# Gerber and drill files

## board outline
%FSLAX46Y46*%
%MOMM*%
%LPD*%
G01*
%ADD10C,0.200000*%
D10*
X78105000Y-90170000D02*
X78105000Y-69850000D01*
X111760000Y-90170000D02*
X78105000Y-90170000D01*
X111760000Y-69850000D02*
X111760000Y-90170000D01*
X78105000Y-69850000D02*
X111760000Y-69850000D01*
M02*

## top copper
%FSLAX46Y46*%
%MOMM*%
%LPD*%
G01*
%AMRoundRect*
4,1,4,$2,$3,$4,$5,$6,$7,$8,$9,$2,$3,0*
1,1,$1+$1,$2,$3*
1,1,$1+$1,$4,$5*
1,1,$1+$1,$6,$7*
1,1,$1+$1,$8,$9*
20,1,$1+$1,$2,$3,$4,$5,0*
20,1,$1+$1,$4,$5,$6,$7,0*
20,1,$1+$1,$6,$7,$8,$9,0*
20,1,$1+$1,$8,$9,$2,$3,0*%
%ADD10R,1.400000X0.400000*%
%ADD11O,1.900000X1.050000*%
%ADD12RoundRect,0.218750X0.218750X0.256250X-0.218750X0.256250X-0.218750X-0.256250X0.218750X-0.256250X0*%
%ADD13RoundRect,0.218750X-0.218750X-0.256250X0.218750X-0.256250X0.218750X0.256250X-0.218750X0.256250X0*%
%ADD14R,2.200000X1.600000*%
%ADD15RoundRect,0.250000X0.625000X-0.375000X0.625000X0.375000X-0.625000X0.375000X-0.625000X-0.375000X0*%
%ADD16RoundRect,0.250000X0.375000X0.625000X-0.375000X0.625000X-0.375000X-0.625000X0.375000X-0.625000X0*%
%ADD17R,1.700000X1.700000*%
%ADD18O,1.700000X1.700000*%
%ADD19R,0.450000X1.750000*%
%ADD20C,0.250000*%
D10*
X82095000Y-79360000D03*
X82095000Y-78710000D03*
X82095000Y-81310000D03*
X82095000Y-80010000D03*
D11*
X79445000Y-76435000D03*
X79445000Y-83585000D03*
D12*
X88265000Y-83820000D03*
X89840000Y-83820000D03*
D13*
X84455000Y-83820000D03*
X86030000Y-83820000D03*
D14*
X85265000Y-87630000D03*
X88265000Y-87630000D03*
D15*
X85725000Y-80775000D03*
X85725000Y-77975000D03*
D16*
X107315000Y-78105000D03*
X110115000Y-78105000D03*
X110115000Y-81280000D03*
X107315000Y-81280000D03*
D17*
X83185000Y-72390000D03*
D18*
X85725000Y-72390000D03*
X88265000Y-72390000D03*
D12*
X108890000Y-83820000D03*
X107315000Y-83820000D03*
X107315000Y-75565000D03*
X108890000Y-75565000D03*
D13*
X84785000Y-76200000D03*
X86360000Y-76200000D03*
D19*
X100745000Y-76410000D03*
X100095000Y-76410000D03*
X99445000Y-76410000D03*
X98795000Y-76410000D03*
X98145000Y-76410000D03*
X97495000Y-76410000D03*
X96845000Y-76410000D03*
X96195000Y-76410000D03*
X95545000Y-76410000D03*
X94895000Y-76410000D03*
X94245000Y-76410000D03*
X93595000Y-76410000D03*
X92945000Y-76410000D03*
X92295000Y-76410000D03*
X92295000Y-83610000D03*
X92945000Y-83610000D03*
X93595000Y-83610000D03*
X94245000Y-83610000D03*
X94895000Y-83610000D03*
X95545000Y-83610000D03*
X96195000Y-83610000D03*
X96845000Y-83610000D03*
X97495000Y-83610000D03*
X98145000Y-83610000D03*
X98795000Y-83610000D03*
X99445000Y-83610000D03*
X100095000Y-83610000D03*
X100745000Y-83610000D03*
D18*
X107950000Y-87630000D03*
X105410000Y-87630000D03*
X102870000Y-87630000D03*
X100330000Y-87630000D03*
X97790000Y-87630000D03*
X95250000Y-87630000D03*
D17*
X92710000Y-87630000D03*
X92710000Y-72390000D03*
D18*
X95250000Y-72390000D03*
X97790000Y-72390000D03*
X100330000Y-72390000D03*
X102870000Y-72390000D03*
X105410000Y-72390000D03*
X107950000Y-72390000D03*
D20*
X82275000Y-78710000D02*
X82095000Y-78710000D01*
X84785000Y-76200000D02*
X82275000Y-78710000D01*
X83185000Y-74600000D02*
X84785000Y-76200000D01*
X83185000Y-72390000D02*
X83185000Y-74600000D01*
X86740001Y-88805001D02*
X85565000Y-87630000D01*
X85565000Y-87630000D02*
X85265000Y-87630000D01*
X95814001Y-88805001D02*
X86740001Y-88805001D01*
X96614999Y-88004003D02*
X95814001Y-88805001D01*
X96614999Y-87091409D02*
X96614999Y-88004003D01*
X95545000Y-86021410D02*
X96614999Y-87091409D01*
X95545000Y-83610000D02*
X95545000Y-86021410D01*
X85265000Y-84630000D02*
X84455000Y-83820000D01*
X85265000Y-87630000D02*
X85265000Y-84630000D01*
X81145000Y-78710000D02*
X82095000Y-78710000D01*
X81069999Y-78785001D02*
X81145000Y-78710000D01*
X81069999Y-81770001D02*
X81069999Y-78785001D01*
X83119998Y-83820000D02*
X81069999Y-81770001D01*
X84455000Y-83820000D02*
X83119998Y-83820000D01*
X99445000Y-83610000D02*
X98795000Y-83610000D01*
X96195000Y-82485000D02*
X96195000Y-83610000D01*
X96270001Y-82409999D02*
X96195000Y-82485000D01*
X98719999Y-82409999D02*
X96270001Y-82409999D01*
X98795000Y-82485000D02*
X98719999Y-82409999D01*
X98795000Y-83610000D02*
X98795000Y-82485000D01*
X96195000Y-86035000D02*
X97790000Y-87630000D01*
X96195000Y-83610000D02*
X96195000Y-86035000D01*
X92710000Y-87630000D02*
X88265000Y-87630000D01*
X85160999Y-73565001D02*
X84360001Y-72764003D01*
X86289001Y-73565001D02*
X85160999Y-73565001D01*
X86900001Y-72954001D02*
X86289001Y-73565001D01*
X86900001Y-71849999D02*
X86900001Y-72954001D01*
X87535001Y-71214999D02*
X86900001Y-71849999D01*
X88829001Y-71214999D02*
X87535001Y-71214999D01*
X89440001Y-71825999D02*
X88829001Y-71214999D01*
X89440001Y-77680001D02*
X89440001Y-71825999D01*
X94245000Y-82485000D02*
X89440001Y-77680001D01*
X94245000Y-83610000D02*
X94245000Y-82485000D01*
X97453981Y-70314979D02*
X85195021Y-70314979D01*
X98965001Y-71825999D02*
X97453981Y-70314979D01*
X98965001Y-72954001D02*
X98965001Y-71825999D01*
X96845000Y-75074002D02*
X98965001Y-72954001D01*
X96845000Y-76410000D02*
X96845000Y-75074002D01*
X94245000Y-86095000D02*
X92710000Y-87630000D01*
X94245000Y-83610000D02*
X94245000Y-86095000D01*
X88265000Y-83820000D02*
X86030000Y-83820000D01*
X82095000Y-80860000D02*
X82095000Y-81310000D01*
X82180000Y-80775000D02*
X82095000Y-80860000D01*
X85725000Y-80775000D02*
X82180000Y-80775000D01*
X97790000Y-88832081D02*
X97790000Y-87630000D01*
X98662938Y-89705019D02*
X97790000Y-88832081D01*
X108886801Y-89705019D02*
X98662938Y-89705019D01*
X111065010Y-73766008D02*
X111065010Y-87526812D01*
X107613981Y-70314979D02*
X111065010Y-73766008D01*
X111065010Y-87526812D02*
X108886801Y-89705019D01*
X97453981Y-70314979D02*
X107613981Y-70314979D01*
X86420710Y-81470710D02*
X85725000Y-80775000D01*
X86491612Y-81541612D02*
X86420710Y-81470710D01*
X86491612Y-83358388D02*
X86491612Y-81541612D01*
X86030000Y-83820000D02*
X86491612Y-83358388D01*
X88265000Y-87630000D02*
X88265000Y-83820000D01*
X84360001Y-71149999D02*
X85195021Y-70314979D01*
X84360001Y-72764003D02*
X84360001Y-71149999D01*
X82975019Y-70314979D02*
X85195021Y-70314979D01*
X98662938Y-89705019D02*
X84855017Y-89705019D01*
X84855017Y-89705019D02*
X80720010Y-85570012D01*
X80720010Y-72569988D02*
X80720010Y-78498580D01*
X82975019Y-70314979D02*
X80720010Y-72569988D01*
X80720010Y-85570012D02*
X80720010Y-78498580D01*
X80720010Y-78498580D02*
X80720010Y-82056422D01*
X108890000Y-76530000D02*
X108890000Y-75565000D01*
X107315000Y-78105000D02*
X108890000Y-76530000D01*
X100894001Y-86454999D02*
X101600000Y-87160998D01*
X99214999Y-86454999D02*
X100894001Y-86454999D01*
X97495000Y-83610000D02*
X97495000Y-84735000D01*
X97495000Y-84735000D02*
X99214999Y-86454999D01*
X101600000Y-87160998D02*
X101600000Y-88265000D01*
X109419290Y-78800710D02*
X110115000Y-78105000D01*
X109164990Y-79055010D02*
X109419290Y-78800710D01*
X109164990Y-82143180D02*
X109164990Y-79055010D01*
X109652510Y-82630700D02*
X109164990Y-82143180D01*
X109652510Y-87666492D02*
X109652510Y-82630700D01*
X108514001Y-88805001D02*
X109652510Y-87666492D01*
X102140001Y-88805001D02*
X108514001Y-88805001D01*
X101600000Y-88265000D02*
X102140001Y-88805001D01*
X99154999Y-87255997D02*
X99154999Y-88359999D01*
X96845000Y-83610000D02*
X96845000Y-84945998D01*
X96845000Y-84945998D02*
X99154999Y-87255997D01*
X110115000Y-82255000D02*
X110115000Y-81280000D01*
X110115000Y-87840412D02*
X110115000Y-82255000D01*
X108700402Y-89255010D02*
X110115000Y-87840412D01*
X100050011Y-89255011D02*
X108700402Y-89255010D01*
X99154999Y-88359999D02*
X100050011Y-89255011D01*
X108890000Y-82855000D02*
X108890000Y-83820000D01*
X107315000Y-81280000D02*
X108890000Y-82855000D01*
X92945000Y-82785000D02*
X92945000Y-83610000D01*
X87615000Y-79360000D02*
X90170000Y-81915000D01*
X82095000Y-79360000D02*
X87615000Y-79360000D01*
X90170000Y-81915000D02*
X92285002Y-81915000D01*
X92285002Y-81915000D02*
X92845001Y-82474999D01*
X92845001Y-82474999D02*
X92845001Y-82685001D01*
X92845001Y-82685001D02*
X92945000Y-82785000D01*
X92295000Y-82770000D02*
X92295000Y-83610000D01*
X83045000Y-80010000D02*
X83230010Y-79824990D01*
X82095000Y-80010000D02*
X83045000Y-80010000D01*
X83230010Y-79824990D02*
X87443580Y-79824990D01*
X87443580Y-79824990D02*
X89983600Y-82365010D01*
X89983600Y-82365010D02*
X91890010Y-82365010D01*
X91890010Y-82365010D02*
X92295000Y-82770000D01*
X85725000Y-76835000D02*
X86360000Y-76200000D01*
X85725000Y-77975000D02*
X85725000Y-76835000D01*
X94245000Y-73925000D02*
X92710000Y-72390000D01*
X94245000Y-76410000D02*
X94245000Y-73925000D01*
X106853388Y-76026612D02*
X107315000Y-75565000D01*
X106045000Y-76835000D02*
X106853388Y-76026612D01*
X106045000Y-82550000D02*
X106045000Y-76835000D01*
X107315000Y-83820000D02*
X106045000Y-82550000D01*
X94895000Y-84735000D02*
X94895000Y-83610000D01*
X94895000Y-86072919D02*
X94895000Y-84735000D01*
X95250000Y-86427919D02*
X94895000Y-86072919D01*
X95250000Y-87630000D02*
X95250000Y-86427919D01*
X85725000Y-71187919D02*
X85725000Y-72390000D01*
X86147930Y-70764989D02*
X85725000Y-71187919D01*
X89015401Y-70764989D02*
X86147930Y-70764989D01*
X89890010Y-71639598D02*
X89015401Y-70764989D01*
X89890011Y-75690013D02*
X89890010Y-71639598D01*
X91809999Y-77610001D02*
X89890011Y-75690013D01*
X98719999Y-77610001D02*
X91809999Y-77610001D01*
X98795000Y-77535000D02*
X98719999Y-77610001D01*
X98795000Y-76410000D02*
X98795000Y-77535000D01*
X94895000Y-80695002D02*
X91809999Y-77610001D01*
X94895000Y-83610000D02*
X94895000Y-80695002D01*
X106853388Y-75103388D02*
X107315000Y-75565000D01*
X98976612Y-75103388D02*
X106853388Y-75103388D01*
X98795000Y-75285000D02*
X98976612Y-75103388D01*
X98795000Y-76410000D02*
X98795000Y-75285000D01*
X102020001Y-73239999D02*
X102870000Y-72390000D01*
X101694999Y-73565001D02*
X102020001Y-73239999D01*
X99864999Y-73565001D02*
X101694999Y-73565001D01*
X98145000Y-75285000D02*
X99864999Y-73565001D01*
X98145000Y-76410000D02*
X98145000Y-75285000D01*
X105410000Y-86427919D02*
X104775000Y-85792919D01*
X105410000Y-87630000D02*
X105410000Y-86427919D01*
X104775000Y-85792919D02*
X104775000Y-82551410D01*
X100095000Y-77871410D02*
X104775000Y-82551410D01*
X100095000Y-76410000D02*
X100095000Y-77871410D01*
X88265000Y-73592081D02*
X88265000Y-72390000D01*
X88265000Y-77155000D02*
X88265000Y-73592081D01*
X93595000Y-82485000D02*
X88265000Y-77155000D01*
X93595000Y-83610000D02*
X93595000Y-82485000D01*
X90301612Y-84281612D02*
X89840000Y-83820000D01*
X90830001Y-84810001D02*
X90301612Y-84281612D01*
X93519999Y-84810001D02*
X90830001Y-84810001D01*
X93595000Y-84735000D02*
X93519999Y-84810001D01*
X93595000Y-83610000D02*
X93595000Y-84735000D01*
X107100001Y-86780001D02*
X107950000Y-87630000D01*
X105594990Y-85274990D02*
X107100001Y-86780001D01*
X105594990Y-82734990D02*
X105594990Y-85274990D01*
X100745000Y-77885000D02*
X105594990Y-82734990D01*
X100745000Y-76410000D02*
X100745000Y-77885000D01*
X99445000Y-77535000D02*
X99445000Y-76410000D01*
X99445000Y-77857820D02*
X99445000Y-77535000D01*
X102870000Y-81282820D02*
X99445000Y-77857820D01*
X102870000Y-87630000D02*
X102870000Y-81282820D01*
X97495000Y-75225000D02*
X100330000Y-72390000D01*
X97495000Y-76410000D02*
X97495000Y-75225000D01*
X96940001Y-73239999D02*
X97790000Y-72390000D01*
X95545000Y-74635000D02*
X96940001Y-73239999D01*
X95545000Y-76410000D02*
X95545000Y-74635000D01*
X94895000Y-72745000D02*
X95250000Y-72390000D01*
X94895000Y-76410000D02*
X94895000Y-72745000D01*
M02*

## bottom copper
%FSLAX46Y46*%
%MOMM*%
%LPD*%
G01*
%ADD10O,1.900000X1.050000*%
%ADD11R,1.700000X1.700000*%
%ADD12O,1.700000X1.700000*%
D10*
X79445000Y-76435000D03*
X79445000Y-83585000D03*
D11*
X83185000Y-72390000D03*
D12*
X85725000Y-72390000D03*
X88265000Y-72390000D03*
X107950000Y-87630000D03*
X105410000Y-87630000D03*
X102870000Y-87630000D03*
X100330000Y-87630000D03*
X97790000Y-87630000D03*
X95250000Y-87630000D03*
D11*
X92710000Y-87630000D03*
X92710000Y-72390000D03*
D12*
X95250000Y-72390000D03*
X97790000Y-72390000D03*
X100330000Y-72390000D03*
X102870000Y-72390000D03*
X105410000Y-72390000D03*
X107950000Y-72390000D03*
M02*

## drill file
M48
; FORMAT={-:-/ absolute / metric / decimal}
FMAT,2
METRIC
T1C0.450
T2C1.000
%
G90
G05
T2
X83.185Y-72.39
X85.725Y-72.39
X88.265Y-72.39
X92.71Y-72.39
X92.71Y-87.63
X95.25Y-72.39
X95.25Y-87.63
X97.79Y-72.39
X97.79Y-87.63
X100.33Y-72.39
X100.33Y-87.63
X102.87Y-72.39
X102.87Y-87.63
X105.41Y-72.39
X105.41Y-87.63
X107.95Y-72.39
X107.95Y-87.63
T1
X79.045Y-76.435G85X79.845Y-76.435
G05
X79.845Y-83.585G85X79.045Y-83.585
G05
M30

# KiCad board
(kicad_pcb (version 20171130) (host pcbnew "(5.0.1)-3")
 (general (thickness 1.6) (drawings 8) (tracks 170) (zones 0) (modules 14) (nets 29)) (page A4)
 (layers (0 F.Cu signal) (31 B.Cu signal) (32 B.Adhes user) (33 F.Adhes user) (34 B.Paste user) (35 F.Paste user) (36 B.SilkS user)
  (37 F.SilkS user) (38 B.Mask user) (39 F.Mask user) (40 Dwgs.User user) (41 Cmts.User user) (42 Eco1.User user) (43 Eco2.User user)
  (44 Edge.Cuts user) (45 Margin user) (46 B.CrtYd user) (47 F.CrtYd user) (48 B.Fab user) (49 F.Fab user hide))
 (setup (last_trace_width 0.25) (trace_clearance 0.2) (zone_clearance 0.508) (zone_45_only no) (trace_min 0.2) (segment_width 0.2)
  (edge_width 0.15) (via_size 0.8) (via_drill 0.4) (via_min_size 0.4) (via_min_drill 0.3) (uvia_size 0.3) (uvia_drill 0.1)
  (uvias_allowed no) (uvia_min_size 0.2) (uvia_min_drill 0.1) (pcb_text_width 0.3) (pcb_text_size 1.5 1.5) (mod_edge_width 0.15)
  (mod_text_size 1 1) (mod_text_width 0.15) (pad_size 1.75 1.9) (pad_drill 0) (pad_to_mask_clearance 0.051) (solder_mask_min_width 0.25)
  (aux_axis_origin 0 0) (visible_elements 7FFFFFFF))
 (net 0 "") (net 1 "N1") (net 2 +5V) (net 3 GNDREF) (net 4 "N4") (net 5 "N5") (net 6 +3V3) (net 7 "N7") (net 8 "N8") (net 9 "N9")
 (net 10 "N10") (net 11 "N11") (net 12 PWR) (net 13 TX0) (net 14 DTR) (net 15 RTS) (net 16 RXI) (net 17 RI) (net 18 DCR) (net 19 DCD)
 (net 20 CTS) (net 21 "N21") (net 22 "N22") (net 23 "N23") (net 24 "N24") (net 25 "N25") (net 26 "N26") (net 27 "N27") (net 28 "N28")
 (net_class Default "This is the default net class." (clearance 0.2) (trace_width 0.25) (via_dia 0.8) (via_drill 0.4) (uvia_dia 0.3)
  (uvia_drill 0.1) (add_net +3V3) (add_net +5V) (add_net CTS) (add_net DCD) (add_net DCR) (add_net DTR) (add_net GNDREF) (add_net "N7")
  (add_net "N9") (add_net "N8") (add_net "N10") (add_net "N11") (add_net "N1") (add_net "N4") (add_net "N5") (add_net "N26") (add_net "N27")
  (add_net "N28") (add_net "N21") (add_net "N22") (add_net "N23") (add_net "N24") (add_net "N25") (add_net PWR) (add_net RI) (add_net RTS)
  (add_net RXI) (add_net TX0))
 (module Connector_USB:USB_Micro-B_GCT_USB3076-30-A (layer F.Cu) (at 80.645 80.01 270)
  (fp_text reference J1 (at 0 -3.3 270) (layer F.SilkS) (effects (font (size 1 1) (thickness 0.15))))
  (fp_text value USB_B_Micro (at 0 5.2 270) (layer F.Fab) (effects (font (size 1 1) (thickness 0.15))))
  (pad 2 smd rect (at -0.65 -1.45 270) (size 0.4 1.4) (layers F.Cu F.Paste F.Mask) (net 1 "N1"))
  (pad 1 smd rect (at -1.3 -1.45 270) (size 0.4 1.4) (layers F.Cu F.Paste F.Mask) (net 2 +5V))
  (pad 5 smd rect (at 1.3 -1.45 270) (size 0.4 1.4) (layers F.Cu F.Paste F.Mask) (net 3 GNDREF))
  (pad 3 smd rect (at 0 -1.45 270) (size 0.4 1.4) (layers F.Cu F.Paste F.Mask) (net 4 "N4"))
  (pad 6 thru_hole oval (at -3.575 1.2 90) (size 1.05 1.9) (drill oval 0.45 1.25) (layers *.Cu *.Mask) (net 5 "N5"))
  (pad 6 thru_hole oval (at 3.575 1.2 270) (size 1.05 1.9) (drill oval 0.45 1.25) (layers *.Cu *.Mask) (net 5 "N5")))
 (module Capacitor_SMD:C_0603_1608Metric (layer F.Cu) (at 89.0525 83.82 180)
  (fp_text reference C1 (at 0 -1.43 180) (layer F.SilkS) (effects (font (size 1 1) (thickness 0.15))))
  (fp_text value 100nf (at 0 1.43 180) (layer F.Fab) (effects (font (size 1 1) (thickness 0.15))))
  (pad 2 smd roundrect (at 0.7875 0 180) (size 0.875 0.95) (layers F.Cu F.Paste F.Mask) (roundrect_rratio 0.25) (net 3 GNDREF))
  (pad 1 smd roundrect (at -0.7875 0 180) (size 0.875 0.95) (layers F.Cu F.Paste F.Mask) (roundrect_rratio 0.25) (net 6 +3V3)))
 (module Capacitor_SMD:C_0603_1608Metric (layer F.Cu) (at 85.2425 83.82)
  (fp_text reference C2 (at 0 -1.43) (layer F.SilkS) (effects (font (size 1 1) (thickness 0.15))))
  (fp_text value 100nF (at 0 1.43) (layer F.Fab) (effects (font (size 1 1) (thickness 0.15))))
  (pad 1 smd roundrect (at -0.7875 0) (size 0.875 0.95) (layers F.Cu F.Paste F.Mask) (roundrect_rratio 0.25) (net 2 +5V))
  (pad 2 smd roundrect (at 0.7875 0) (size 0.875 0.95) (layers F.Cu F.Paste F.Mask) (roundrect_rratio 0.25) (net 3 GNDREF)))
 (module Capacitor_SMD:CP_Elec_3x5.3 (layer F.Cu) (at 86.765 87.63)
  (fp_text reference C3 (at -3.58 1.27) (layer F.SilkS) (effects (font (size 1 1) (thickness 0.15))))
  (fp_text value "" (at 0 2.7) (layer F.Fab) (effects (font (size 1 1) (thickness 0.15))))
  (pad 1 smd rect (at -1.5 0) (size 2.2 1.6) (layers F.Cu F.Paste F.Mask) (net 2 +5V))
  (pad 2 smd rect (at 1.5 0) (size 2.2 1.6) (layers F.Cu F.Paste F.Mask) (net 3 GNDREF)))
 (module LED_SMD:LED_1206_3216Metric (layer F.Cu) (at 85.725 79.375 90)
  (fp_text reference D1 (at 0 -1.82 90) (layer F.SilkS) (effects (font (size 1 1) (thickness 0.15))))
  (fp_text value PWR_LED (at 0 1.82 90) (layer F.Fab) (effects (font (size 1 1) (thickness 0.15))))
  (pad 1 smd roundrect (at -1.4 0 90) (size 1.25 1.75) (layers F.Cu F.Paste F.Mask) (roundrect_rratio 0.2) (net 3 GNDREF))
  (pad 2 smd roundrect (at 1.4 0 90) (size 1.25 1.75) (layers F.Cu F.Paste F.Mask) (roundrect_rratio 0.2) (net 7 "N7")))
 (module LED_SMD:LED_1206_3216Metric (layer F.Cu) (at 108.715 78.105 180)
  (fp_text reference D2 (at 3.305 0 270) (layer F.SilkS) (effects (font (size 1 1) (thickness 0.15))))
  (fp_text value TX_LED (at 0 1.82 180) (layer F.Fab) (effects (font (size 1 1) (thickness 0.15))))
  (pad 2 smd roundrect (at 1.4 0 180) (size 1.25 1.75) (layers F.Cu F.Paste F.Mask) (roundrect_rratio 0.2) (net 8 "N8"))
  (pad 1 smd roundrect (at -1.4 0 180) (size 1.25 1.75) (layers F.Cu F.Paste F.Mask) (roundrect_rratio 0.2) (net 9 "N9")))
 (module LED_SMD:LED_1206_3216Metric (layer F.Cu) (at 108.715 81.28 180)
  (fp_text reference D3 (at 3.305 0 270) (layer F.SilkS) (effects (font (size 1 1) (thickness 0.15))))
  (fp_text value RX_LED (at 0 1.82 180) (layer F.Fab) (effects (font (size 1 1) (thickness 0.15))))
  (pad 1 smd roundrect (at -1.4 0 180) (size 1.25 1.75) (layers F.Cu F.Paste F.Mask) (roundrect_rratio 0.2) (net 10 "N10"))
  (pad 2 smd roundrect (at 1.4 0 180) (size 1.25 1.75) (layers F.Cu F.Paste F.Mask) (roundrect_rratio 0.2) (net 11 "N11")))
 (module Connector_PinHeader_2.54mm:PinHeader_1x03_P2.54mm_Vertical (layer F.Cu) (at 83.185 72.39 90)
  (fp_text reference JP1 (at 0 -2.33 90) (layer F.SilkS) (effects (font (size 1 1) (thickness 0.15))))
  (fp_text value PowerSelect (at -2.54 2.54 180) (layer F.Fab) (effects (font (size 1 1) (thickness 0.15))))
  (pad 1 thru_hole rect (at 0 0 90) (size 1.7 1.7) (drill 1) (layers *.Cu *.Mask) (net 2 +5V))
  (pad 2 thru_hole oval (at 0 2.54 90) (size 1.7 1.7) (drill 1) (layers *.Cu *.Mask) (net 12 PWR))
  (pad 3 thru_hole oval (at 0 5.08 90) (size 1.7 1.7) (drill 1) (layers *.Cu *.Mask) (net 6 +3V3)))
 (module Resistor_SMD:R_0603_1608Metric (layer F.Cu) (at 108.1025 83.82 180)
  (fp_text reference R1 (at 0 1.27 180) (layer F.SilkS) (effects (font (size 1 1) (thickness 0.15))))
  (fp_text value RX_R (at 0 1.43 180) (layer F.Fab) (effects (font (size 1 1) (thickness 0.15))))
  (pad 1 smd roundrect (at -0.7875 0 180) (size 0.875 0.95) (layers F.Cu F.Paste F.Mask) (roundrect_rratio 0.25) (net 11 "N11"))
  (pad 2 smd roundrect (at 0.7875 0 180) (size 0.875 0.95) (layers F.Cu F.Paste F.Mask) (roundrect_rratio 0.25) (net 12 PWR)))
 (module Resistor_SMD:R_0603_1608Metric (layer F.Cu) (at 108.1025 75.565 180)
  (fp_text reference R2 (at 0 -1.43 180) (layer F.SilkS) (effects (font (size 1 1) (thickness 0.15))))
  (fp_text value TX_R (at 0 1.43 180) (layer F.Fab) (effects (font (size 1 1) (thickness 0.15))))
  (pad 2 smd roundrect (at 0.7875 0 180) (size 0.875 0.95) (layers F.Cu F.Paste F.Mask) (roundrect_rratio 0.25) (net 12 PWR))
  (pad 1 smd roundrect (at -0.7875 0 180) (size 0.875 0.95) (layers F.Cu F.Paste F.Mask) (roundrect_rratio 0.25) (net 8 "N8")))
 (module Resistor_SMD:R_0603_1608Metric (layer F.Cu) (at 85.5725 76.2)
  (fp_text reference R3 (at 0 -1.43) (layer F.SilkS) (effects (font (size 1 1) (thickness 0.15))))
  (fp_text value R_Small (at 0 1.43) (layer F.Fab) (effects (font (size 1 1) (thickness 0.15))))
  (pad 1 smd roundrect (at -0.7875 0) (size 0.875 0.95) (layers F.Cu F.Paste F.Mask) (roundrect_rratio 0.25) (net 2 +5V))
  (pad 2 smd roundrect (at 0.7875 0) (size 0.875 0.95) (layers F.Cu F.Paste F.Mask) (roundrect_rratio 0.25) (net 7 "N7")))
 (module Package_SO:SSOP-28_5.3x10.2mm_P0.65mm (layer F.Cu) (at 96.52 80.01 270)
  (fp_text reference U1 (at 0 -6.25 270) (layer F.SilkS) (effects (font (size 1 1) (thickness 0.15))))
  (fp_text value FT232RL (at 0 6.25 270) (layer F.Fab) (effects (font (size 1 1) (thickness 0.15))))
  (pad 1 smd rect (at -3.6 -4.225 270) (size 1.75 0.45) (layers F.Cu F.Paste F.Mask) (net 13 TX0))
  (pad 2 smd rect (at -3.6 -3.575 270) (size 1.75 0.45) (layers F.Cu F.Paste F.Mask) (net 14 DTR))
  (pad 3 smd rect (at -3.6 -2.925 270) (size 1.75 0.45) (layers F.Cu F.Paste F.Mask) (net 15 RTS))
  (pad 4 smd rect (at -3.6 -2.275 270) (size 1.75 0.45) (layers F.Cu F.Paste F.Mask) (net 12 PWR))
  (pad 5 smd rect (at -3.6 -1.625 270) (size 1.75 0.45) (layers F.Cu F.Paste F.Mask) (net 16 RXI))
  (pad 6 smd rect (at -3.6 -0.975 270) (size 1.75 0.45) (layers F.Cu F.Paste F.Mask) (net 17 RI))
  (pad 7 smd rect (at -3.6 -0.325 270) (size 1.75 0.45) (layers F.Cu F.Paste F.Mask) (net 3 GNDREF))
  (pad 8 smd rect (at -3.6 0.325 270) (size 1.75 0.45) (layers F.Cu F.Paste F.Mask))
  (pad 9 smd rect (at -3.6 0.975 270) (size 1.75 0.45) (layers F.Cu F.Paste F.Mask) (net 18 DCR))
  (pad 10 smd rect (at -3.6 1.625 270) (size 1.75 0.45) (layers F.Cu F.Paste F.Mask) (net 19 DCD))
  (pad 11 smd rect (at -3.6 2.275 270) (size 1.75 0.45) (layers F.Cu F.Paste F.Mask) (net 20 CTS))
  (pad 12 smd rect (at -3.6 2.925 270) (size 1.75 0.45) (layers F.Cu F.Paste F.Mask) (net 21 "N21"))
  (pad 13 smd rect (at -3.6 3.575 270) (size 1.75 0.45) (layers F.Cu F.Paste F.Mask) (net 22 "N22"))
  (pad 14 smd rect (at -3.6 4.225 270) (size 1.75 0.45) (layers F.Cu F.Paste F.Mask) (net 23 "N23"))
  (pad 15 smd rect (at 3.6 4.225 270) (size 1.75 0.45) (layers F.Cu F.Paste F.Mask) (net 4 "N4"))
  (pad 16 smd rect (at 3.6 3.575 270) (size 1.75 0.45) (layers F.Cu F.Paste F.Mask) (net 1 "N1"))
  (pad 17 smd rect (at 3.6 2.925 270) (size 1.75 0.45) (layers F.Cu F.Paste F.Mask) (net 6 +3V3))
  (pad 18 smd rect (at 3.6 2.275 270) (size 1.75 0.45) (layers F.Cu F.Paste F.Mask) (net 3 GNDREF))
  (pad 19 smd rect (at 3.6 1.625 270) (size 1.75 0.45) (layers F.Cu F.Paste F.Mask) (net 12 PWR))
  (pad 20 smd rect (at 3.6 0.975 270) (size 1.75 0.45) (layers F.Cu F.Paste F.Mask) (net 2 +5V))
  (pad 21 smd rect (at 3.6 0.325 270) (size 1.75 0.45) (layers F.Cu F.Paste F.Mask) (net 3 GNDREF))
  (pad 22 smd rect (at 3.6 -0.325 270) (size 1.75 0.45) (layers F.Cu F.Paste F.Mask) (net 10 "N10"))
  (pad 23 smd rect (at 3.6 -0.975 270) (size 1.75 0.45) (layers F.Cu F.Paste F.Mask) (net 9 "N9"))
  (pad 24 smd rect (at 3.6 -1.625 270) (size 1.75 0.45) (layers F.Cu F.Paste F.Mask))
  (pad 25 smd rect (at 3.6 -2.275 270) (size 1.75 0.45) (layers F.Cu F.Paste F.Mask) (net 3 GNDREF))
  (pad 26 smd rect (at 3.6 -2.925 270) (size 1.75 0.45) (layers F.Cu F.Paste F.Mask) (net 3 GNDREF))
  (pad 27 smd rect (at 3.6 -3.575 270) (size 1.75 0.45) (layers F.Cu F.Paste F.Mask) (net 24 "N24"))
  (pad 28 smd rect (at 3.6 -4.225 270) (size 1.75 0.45) (layers F.Cu F.Paste F.Mask) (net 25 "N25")))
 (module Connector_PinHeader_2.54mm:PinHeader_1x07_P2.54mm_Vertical (layer F.Cu) (at 92.71 87.63 90)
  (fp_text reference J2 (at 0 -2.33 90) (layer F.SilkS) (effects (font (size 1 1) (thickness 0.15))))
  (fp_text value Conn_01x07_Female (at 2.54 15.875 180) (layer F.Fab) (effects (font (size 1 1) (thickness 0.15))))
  (pad 7 thru_hole oval (at 0 15.24 90) (size 1.7 1.7) (drill 1) (layers *.Cu *.Mask) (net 13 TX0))
  (pad 6 thru_hole oval (at 0 12.7 90) (size 1.7 1.7) (drill 1) (layers *.Cu *.Mask) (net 14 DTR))
  (pad 5 thru_hole oval (at 0 10.16 90) (size 1.7 1.7) (drill 1) (layers *.Cu *.Mask) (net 15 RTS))
  (pad 4 thru_hole oval (at 0 7.62 90) (size 1.7 1.7) (drill 1) (layers *.Cu *.Mask) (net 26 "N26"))
  (pad 3 thru_hole oval (at 0 5.08 90) (size 1.7 1.7) (drill 1) (layers *.Cu *.Mask) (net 3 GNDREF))
  (pad 2 thru_hole oval (at 0 2.54 90) (size 1.7 1.7) (drill 1) (layers *.Cu *.Mask) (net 12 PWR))
  (pad 1 thru_hole rect (at 0 0 90) (size 1.7 1.7) (drill 1) (layers *.Cu *.Mask) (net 3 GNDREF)))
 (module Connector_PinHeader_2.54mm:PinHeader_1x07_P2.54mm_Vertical (layer F.Cu) (at 92.71 72.39 90)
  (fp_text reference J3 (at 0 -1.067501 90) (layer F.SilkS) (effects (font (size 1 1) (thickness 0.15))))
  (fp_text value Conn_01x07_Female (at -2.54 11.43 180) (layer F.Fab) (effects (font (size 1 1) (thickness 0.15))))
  (pad 1 thru_hole rect (at 0 0 90) (size 1.7 1.7) (drill 1) (layers *.Cu *.Mask) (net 20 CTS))
  (pad 2 thru_hole oval (at 0 2.54 90) (size 1.7 1.7) (drill 1) (layers *.Cu *.Mask) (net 19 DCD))
  (pad 3 thru_hole oval (at 0 5.08 90) (size 1.7 1.7) (drill 1) (layers *.Cu *.Mask) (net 18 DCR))
  (pad 4 thru_hole oval (at 0 7.62 90) (size 1.7 1.7) (drill 1) (layers *.Cu *.Mask) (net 17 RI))
  (pad 5 thru_hole oval (at 0 10.16 90) (size 1.7 1.7) (drill 1) (layers *.Cu *.Mask) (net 16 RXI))
  (pad 6 thru_hole oval (at 0 12.7 90) (size 1.7 1.7) (drill 1) (layers *.Cu *.Mask) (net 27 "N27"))
  (pad 7 thru_hole oval (at 0 15.24 90) (size 1.7 1.7) (drill 1) (layers *.Cu *.Mask) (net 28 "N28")))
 (gr_line (start 78.105 90.17) (end 78.105 69.85) (layer Edge.Cuts) (width 0.2))
 (gr_line (start 111.76 90.17) (end 78.105 90.17) (layer Edge.Cuts) (width 0.2))
 (gr_line (start 111.76 69.85) (end 111.76 90.17) (layer Edge.Cuts) (width 0.2))
 (gr_line (start 78.105 69.85) (end 111.76 69.85) (layer Edge.Cuts) (width 0.2))
 (segment (start 82.275 78.71) (end 82.095 78.71) (width 0.25) (layer F.Cu) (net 2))
 (segment (start 84.785 76.2) (end 82.275 78.71) (width 0.25) (layer F.Cu) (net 2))
 (segment (start 83.185 74.6) (end 84.785 76.2) (width 0.25) (layer F.Cu) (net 2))
 (segment (start 83.185 72.39) (end 83.185 74.6) (width 0.25) (layer F.Cu) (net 2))
 (segment (start 86.740001 88.805001) (end 85.565 87.63) (width 0.25) (layer F.Cu) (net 2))
 (segment (start 85.565 87.63) (end 85.265 87.63) (width 0.25) (layer F.Cu) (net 2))
 (segment (start 95.814001 88.805001) (end 86.740001 88.805001) (width 0.25) (layer F.Cu) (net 2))
 (segment (start 96.614999 88.004003) (end 95.814001 88.805001) (width 0.25) (layer F.Cu) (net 2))
 (segment (start 96.614999 87.091409) (end 96.614999 88.004003) (width 0.25) (layer F.Cu) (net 2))
 (segment (start 95.545 86.02141) (end 96.614999 87.091409) (width 0.25) (layer F.Cu) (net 2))
 (segment (start 95.545 83.61) (end 95.545 86.02141) (width 0.25) (layer F.Cu) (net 2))
 (segment (start 85.265 84.63) (end 84.455 83.82) (width 0.25) (layer F.Cu) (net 2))
 (segment (start 85.265 87.63) (end 85.265 84.63) (width 0.25) (layer F.Cu) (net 2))
 (segment (start 81.145 78.71) (end 82.095 78.71) (width 0.25) (layer F.Cu) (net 2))
 (segment (start 81.069999 78.785001) (end 81.145 78.71) (width 0.25) (layer F.Cu) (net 2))
 (segment (start 81.069999 81.770001) (end 81.069999 78.785001) (width 0.25) (layer F.Cu) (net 2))
 (segment (start 83.119998 83.82) (end 81.069999 81.770001) (width 0.25) (layer F.Cu) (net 2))
 (segment (start 84.455 83.82) (end 83.119998 83.82) (width 0.25) (layer F.Cu) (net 2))
 (segment (start 99.445 83.61) (end 98.795 83.61) (width 0.25) (layer F.Cu) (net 3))
 (segment (start 96.195 82.485) (end 96.195 83.61) (width 0.25) (layer F.Cu) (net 3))
 (segment (start 96.270001 82.409999) (end 96.195 82.485) (width 0.25) (layer F.Cu) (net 3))
 (segment (start 98.719999 82.409999) (end 96.270001 82.409999) (width 0.25) (layer F.Cu) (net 3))
 (segment (start 98.795 82.485) (end 98.719999 82.409999) (width 0.25) (layer F.Cu) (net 3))
 (segment (start 98.795 83.61) (end 98.795 82.485) (width 0.25) (layer F.Cu) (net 3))
 (segment (start 96.195 86.035) (end 97.79 87.63) (width 0.25) (layer F.Cu) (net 3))
 (segment (start 96.195 83.61) (end 96.195 86.035) (width 0.25) (layer F.Cu) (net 3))
 (segment (start 92.71 87.63) (end 88.265 87.63) (width 0.25) (layer F.Cu) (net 3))
 (segment (start 85.160999 73.565001) (end 84.360001 72.764003) (width 0.25) (layer F.Cu) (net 3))
 (segment (start 86.289001 73.565001) (end 85.160999 73.565001) (width 0.25) (layer F.Cu) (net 3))
 (segment (start 86.900001 72.954001) (end 86.289001 73.565001) (width 0.25) (layer F.Cu) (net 3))
 (segment (start 86.900001 71.849999) (end 86.900001 72.954001) (width 0.25) (layer F.Cu) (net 3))
 (segment (start 87.535001 71.214999) (end 86.900001 71.849999) (width 0.25) (layer F.Cu) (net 3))
 (segment (start 88.829001 71.214999) (end 87.535001 71.214999) (width 0.25) (layer F.Cu) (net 3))
 (segment (start 89.440001 71.825999) (end 88.829001 71.214999) (width 0.25) (layer F.Cu) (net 3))
 (segment (start 89.440001 77.680001) (end 89.440001 71.825999) (width 0.25) (layer F.Cu) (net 3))
 (segment (start 94.245 82.485) (end 89.440001 77.680001) (width 0.25) (layer F.Cu) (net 3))
 (segment (start 94.245 83.61) (end 94.245 82.485) (width 0.25) (layer F.Cu) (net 3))
 (segment (start 97.453981 70.314979) (end 85.195021 70.314979) (width 0.25) (layer F.Cu) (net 3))
 (segment (start 98.965001 71.825999) (end 97.453981 70.314979) (width 0.25) (layer F.Cu) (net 3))
 (segment (start 98.965001 72.954001) (end 98.965001 71.825999) (width 0.25) (layer F.Cu) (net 3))
 (segment (start 96.845 75.074002) (end 98.965001 72.954001) (width 0.25) (layer F.Cu) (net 3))
 (segment (start 96.845 76.41) (end 96.845 75.074002) (width 0.25) (layer F.Cu) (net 3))
 (segment (start 94.245 86.095) (end 92.71 87.63) (width 0.25) (layer F.Cu) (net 3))
 (segment (start 94.245 83.61) (end 94.245 86.095) (width 0.25) (layer F.Cu) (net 3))
 (segment (start 88.265 83.82) (end 86.03 83.82) (width 0.25) (layer F.Cu) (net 3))
 (segment (start 82.095 80.86) (end 82.095 81.31) (width 0.25) (layer F.Cu) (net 3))
 (segment (start 82.18 80.775) (end 82.095 80.86) (width 0.25) (layer F.Cu) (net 3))
 (segment (start 85.725 80.775) (end 82.18 80.775) (width 0.25) (layer F.Cu) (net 3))
 (segment (start 97.79 88.832081) (end 97.79 87.63) (width 0.25) (layer F.Cu) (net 3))
 (segment (start 98.662938 89.705019) (end 97.79 88.832081) (width 0.25) (layer F.Cu) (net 3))
 (segment (start 108.886801 89.705019) (end 98.662938 89.705019) (width 0.25) (layer F.Cu) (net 3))
 (segment (start 111.06501 73.766008) (end 111.06501 87.526812) (width 0.25) (layer F.Cu) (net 3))
 (segment (start 107.613981 70.314979) (end 111.06501 73.766008) (width 0.25) (layer F.Cu) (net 3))
 (segment (start 111.06501 87.526812) (end 108.886801 89.705019) (width 0.25) (layer F.Cu) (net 3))
 (segment (start 97.453981 70.314979) (end 107.613981 70.314979) (width 0.25) (layer F.Cu) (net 3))
 (segment (start 86.42071 81.47071) (end 85.725 80.775) (width 0.25) (layer F.Cu) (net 3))
 (segment (start 86.491612 81.541612) (end 86.42071 81.47071) (width 0.25) (layer F.Cu) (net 3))
 (segment (start 86.491612 83.358388) (end 86.491612 81.541612) (width 0.25) (layer F.Cu) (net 3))
 (segment (start 86.03 83.82) (end 86.491612 83.358388) (width 0.25) (layer F.Cu) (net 3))
 (segment (start 88.265 87.63) (end 88.265 83.82) (width 0.25) (layer F.Cu) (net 3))
 (segment (start 84.360001 71.149999) (end 85.195021 70.314979) (width 0.25) (layer F.Cu) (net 3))
 (segment (start 84.360001 72.764003) (end 84.360001 71.149999) (width 0.25) (layer F.Cu) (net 3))
 (segment (start 82.975019 70.314979) (end 85.195021 70.314979) (width 0.25) (layer F.Cu) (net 3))
 (segment (start 98.662938 89.705019) (end 84.855017 89.705019) (width 0.25) (layer F.Cu) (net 3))
 (segment (start 84.855017 89.705019) (end 80.72001 85.570012) (width 0.25) (layer F.Cu) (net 3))
 (segment (start 80.72001 72.569988) (end 80.72001 78.49858) (width 0.25) (layer F.Cu) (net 3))
 (segment (start 82.975019 70.314979) (end 80.72001 72.569988) (width 0.25) (layer F.Cu) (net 3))
 (segment (start 80.72001 85.570012) (end 80.72001 78.49858) (width 0.25) (layer F.Cu) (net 3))
 (segment (start 80.72001 78.49858) (end 80.72001 82.056422) (width 0.25) (layer F.Cu) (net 3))
 (segment (start 108.89 76.53) (end 108.89 75.565) (width 0.25) (layer F.Cu) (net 8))
 (segment (start 107.315 78.105) (end 108.89 76.53) (width 0.25) (layer F.Cu) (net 8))
 (segment (start 100.894001 86.454999) (end 101.6 87.160998) (width 0.25) (layer F.Cu) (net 9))
 (segment (start 99.214999 86.454999) (end 100.894001 86.454999) (width 0.25) (layer F.Cu) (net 9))
 (segment (start 97.495 83.61) (end 97.495 84.735) (width 0.25) (layer F.Cu) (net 9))
 (segment (start 97.495 84.735) (end 99.214999 86.454999) (width 0.25) (layer F.Cu) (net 9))
 (segment (start 101.6 87.160998) (end 101.6 88.265) (width 0.25) (layer F.Cu) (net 9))
 (segment (start 109.41929 78.80071) (end 110.115 78.105) (width 0.25) (layer F.Cu) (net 9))
 (segment (start 109.16499 79.05501) (end 109.41929 78.80071) (width 0.25) (layer F.Cu) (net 9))
 (segment (start 109.16499 82.14318) (end 109.16499 79.05501) (width 0.25) (layer F.Cu) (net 9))
 (segment (start 109.65251 82.6307) (end 109.16499 82.14318) (width 0.25) (layer F.Cu) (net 9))
 (segment (start 109.65251 87.666492) (end 109.65251 82.6307) (width 0.25) (layer F.Cu) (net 9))
 (segment (start 108.514001 88.805001) (end 109.65251 87.666492) (width 0.25) (layer F.Cu) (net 9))
 (segment (start 102.140001 88.805001) (end 108.514001 88.805001) (width 0.25) (layer F.Cu) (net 9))
 (segment (start 101.6 88.265) (end 102.140001 88.805001) (width 0.25) (layer F.Cu) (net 9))
 (segment (start 99.154999 87.255997) (end 99.154999 88.359999) (width 0.25) (layer F.Cu) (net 10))
 (segment (start 96.845 83.61) (end 96.845 84.945998) (width 0.25) (layer F.Cu) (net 10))
 (segment (start 96.845 84.945998) (end 99.154999 87.255997) (width 0.25) (layer F.Cu) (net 10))
 (segment (start 110.115 82.255) (end 110.115 81.28) (width 0.25) (layer F.Cu) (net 10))
 (segment (start 110.115 87.840412) (end 110.115 82.255) (width 0.25) (layer F.Cu) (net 10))
 (segment (start 108.700402 89.25501) (end 110.115 87.840412) (width 0.25) (layer F.Cu) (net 10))
 (segment (start 100.050011 89.255011) (end 108.700402 89.25501) (width 0.25) (layer F.Cu) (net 10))
 (segment (start 99.154999 88.359999) (end 100.050011 89.255011) (width 0.25) (layer F.Cu) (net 10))
 (segment (start 108.89 82.855) (end 108.89 83.82) (width 0.25) (layer F.Cu) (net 11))
 (segment (start 107.315 81.28) (end 108.89 82.855) (width 0.25) (layer F.Cu) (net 11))
 (segment (start 92.945 82.785) (end 92.945 83.61) (width 0.25) (layer F.Cu) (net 1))
 (segment (start 87.615 79.36) (end 90.17 81.915) (width 0.25) (layer F.Cu) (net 1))
 (segment (start 82.095 79.36) (end 87.615 79.36) (width 0.25) (layer F.Cu) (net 1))
 (segment (start 90.17 81.915) (end 92.285002 81.915) (width 0.25) (layer F.Cu) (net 1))
 (segment (start 92.285002 81.915) (end 92.845001 82.474999) (width 0.25) (layer F.Cu) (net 1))
 (segment (start 92.845001 82.474999) (end 92.845001 82.685001) (width 0.25) (layer F.Cu) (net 1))
 (segment (start 92.845001 82.685001) (end 92.945 82.785) (width 0.25) (layer F.Cu) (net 1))
 (segment (start 92.295 82.77) (end 92.295 83.61) (width 0.25) (layer F.Cu) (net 4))
 (segment (start 83.045 80.01) (end 83.23001 79.82499) (width 0.25) (layer F.Cu) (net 4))
 (segment (start 82.095 80.01) (end 83.045 80.01) (width 0.25) (layer F.Cu) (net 4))
 (segment (start 83.23001 79.82499) (end 87.44358 79.82499) (width 0.25) (layer F.Cu) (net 4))
 (segment (start 87.44358 79.82499) (end 89.9836 82.36501) (width 0.25) (layer F.Cu) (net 4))
 (segment (start 89.9836 82.36501) (end 91.89001 82.36501) (width 0.25) (layer F.Cu) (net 4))
 (segment (start 91.89001 82.36501) (end 92.295 82.77) (width 0.25) (layer F.Cu) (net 4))
 (segment (start 85.725 76.835) (end 86.36 76.2) (width 0.25) (layer F.Cu) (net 7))
 (segment (start 85.725 77.975) (end 85.725 76.835) (width 0.25) (layer F.Cu) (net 7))
 (segment (start 94.245 73.925) (end 92.71 72.39) (width 0.25) (layer F.Cu) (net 20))
 (segment (start 94.245 76.41) (end 94.245 73.925) (width 0.25) (layer F.Cu) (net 20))
 (segment (start 106.853388 76.026612) (end 107.315 75.565) (width 0.25) (layer F.Cu) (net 12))
 (segment (start 106.045 76.835) (end 106.853388 76.026612) (width 0.25) (layer F.Cu) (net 12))
 (segment (start 106.045 82.55) (end 106.045 76.835) (width 0.25) (layer F.Cu) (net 12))
 (segment (start 107.315 83.82) (end 106.045 82.55) (width 0.25) (layer F.Cu) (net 12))
 (segment (start 94.895 84.735) (end 94.895 83.61) (width 0.25) (layer F.Cu) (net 12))
 (segment (start 94.895 86.072919) (end 94.895 84.735) (width 0.25) (layer F.Cu) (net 12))
 (segment (start 95.25 86.427919) (end 94.895 86.072919) (width 0.25) (layer F.Cu) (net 12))
 (segment (start 95.25 87.63) (end 95.25 86.427919) (width 0.25) (layer F.Cu) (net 12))
 (segment (start 85.725 71.187919) (end 85.725 72.39) (width 0.25) (layer F.Cu) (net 12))
 (segment (start 86.14793 70.764989) (end 85.725 71.187919) (width 0.25) (layer F.Cu) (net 12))
 (segment (start 89.015401 70.764989) (end 86.14793 70.764989) (width 0.25) (layer F.Cu) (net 12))
 (segment (start 89.89001 71.639598) (end 89.015401 70.764989) (width 0.25) (layer F.Cu) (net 12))
 (segment (start 89.890011 75.690013) (end 89.89001 71.639598) (width 0.25) (layer F.Cu) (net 12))
 (segment (start 91.809999 77.610001) (end 89.890011 75.690013) (width 0.25) (layer F.Cu) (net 12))
 (segment (start 98.719999 77.610001) (end 91.809999 77.610001) (width 0.25) (layer F.Cu) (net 12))
 (segment (start 98.795 77.535) (end 98.719999 77.610001) (width 0.25) (layer F.Cu) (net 12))
 (segment (start 98.795 76.41) (end 98.795 77.535) (width 0.25) (layer F.Cu) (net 12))
 (segment (start 94.895 80.695002) (end 91.809999 77.610001) (width 0.25) (layer F.Cu) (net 12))
 (segment (start 94.895 83.61) (end 94.895 80.695002) (width 0.25) (layer F.Cu) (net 12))
 (segment (start 106.853388 75.103388) (end 107.315 75.565) (width 0.25) (layer F.Cu) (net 12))
 (segment (start 98.976612 75.103388) (end 106.853388 75.103388) (width 0.25) (layer F.Cu) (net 12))
 (segment (start 98.795 75.285) (end 98.976612 75.103388) (width 0.25) (layer F.Cu) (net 12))
 (segment (start 98.795 76.41) (end 98.795 75.285) (width 0.25) (layer F.Cu) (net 12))
 (segment (start 102.020001 73.239999) (end 102.87 72.39) (width 0.25) (layer F.Cu) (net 16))
 (segment (start 101.694999 73.565001) (end 102.020001 73.239999) (width 0.25) (layer F.Cu) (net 16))
 (segment (start 99.864999 73.565001) (end 101.694999 73.565001) (width 0.25) (layer F.Cu) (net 16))
 (segment (start 98.145 75.285) (end 99.864999 73.565001) (width 0.25) (layer F.Cu) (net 16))
 (segment (start 98.145 76.41) (end 98.145 75.285) (width 0.25) (layer F.Cu) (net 16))
 (segment (start 105.41 86.427919) (end 104.775 85.792919) (width 0.25) (layer F.Cu) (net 14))
 (segment (start 105.41 87.63) (end 105.41 86.427919) (width 0.25) (layer F.Cu) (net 14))
 (segment (start 104.775 85.792919) (end 104.775 82.55141) (width 0.25) (layer F.Cu) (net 14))
 (segment (start 100.095 77.87141) (end 104.775 82.55141) (width 0.25) (layer F.Cu) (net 14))
 (segment (start 100.095 76.41) (end 100.095 77.87141) (width 0.25) (layer F.Cu) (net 14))
 (segment (start 88.265 73.592081) (end 88.265 72.39) (width 0.25) (layer F.Cu) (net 6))
 (segment (start 88.265 77.155) (end 88.265 73.592081) (width 0.25) (layer F.Cu) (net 6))
 (segment (start 93.595 82.485) (end 88.265 77.155) (width 0.25) (layer F.Cu) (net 6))
 (segment (start 93.595 83.61) (end 93.595 82.485) (width 0.25) (layer F.Cu) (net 6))
 (segment (start 90.301612 84.281612) (end 89.84 83.82) (width 0.25) (layer F.Cu) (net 6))
 (segment (start 90.830001 84.810001) (end 90.301612 84.281612) (width 0.25) (layer F.Cu) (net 6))
 (segment (start 93.519999 84.810001) (end 90.830001 84.810001) (width 0.25) (layer F.Cu) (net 6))
 (segment (start 93.595 84.735) (end 93.519999 84.810001) (width 0.25) (layer F.Cu) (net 6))
 (segment (start 93.595 83.61) (end 93.595 84.735) (width 0.25) (layer F.Cu) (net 6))
 (segment (start 107.100001 86.780001) (end 107.95 87.63) (width 0.25) (layer F.Cu) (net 13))
 (segment (start 105.59499 85.27499) (end 107.100001 86.780001) (width 0.25) (layer F.Cu) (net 13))
 (segment (start 105.59499 82.73499) (end 105.59499 85.27499) (width 0.25) (layer F.Cu) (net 13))
 (segment (start 100.745 77.885) (end 105.59499 82.73499) (width 0.25) (layer F.Cu) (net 13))
 (segment (start 100.745 76.41) (end 100.745 77.885) (width 0.25) (layer F.Cu) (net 13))
 (segment (start 99.445 77.535) (end 99.445 76.41) (width 0.25) (layer F.Cu) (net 15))
 (segment (start 99.445 77.85782) (end 99.445 77.535) (width 0.25) (layer F.Cu) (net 15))
 (segment (start 102.87 81.28282) (end 99.445 77.85782) (width 0.25) (layer F.Cu) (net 15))
 (segment (start 102.87 87.63) (end 102.87 81.28282) (width 0.25) (layer F.Cu) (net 15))
 (segment (start 97.495 75.225) (end 100.33 72.39) (width 0.25) (layer F.Cu) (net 17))
 (segment (start 97.495 76.41) (end 97.495 75.225) (width 0.25) (layer F.Cu) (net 17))
 (segment (start 96.940001 73.239999) (end 97.79 72.39) (width 0.25) (layer F.Cu) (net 18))
 (segment (start 95.545 74.635) (end 96.940001 73.239999) (width 0.25) (layer F.Cu) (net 18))
 (segment (start 95.545 76.41) (end 95.545 74.635) (width 0.25) (layer F.Cu) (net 18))
 (segment (start 94.895 72.745) (end 95.25 72.39) (width 0.25) (layer F.Cu) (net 19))
 (segment (start 94.895 76.41) (end 94.895 72.745) (width 0.25) (layer F.Cu) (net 19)))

